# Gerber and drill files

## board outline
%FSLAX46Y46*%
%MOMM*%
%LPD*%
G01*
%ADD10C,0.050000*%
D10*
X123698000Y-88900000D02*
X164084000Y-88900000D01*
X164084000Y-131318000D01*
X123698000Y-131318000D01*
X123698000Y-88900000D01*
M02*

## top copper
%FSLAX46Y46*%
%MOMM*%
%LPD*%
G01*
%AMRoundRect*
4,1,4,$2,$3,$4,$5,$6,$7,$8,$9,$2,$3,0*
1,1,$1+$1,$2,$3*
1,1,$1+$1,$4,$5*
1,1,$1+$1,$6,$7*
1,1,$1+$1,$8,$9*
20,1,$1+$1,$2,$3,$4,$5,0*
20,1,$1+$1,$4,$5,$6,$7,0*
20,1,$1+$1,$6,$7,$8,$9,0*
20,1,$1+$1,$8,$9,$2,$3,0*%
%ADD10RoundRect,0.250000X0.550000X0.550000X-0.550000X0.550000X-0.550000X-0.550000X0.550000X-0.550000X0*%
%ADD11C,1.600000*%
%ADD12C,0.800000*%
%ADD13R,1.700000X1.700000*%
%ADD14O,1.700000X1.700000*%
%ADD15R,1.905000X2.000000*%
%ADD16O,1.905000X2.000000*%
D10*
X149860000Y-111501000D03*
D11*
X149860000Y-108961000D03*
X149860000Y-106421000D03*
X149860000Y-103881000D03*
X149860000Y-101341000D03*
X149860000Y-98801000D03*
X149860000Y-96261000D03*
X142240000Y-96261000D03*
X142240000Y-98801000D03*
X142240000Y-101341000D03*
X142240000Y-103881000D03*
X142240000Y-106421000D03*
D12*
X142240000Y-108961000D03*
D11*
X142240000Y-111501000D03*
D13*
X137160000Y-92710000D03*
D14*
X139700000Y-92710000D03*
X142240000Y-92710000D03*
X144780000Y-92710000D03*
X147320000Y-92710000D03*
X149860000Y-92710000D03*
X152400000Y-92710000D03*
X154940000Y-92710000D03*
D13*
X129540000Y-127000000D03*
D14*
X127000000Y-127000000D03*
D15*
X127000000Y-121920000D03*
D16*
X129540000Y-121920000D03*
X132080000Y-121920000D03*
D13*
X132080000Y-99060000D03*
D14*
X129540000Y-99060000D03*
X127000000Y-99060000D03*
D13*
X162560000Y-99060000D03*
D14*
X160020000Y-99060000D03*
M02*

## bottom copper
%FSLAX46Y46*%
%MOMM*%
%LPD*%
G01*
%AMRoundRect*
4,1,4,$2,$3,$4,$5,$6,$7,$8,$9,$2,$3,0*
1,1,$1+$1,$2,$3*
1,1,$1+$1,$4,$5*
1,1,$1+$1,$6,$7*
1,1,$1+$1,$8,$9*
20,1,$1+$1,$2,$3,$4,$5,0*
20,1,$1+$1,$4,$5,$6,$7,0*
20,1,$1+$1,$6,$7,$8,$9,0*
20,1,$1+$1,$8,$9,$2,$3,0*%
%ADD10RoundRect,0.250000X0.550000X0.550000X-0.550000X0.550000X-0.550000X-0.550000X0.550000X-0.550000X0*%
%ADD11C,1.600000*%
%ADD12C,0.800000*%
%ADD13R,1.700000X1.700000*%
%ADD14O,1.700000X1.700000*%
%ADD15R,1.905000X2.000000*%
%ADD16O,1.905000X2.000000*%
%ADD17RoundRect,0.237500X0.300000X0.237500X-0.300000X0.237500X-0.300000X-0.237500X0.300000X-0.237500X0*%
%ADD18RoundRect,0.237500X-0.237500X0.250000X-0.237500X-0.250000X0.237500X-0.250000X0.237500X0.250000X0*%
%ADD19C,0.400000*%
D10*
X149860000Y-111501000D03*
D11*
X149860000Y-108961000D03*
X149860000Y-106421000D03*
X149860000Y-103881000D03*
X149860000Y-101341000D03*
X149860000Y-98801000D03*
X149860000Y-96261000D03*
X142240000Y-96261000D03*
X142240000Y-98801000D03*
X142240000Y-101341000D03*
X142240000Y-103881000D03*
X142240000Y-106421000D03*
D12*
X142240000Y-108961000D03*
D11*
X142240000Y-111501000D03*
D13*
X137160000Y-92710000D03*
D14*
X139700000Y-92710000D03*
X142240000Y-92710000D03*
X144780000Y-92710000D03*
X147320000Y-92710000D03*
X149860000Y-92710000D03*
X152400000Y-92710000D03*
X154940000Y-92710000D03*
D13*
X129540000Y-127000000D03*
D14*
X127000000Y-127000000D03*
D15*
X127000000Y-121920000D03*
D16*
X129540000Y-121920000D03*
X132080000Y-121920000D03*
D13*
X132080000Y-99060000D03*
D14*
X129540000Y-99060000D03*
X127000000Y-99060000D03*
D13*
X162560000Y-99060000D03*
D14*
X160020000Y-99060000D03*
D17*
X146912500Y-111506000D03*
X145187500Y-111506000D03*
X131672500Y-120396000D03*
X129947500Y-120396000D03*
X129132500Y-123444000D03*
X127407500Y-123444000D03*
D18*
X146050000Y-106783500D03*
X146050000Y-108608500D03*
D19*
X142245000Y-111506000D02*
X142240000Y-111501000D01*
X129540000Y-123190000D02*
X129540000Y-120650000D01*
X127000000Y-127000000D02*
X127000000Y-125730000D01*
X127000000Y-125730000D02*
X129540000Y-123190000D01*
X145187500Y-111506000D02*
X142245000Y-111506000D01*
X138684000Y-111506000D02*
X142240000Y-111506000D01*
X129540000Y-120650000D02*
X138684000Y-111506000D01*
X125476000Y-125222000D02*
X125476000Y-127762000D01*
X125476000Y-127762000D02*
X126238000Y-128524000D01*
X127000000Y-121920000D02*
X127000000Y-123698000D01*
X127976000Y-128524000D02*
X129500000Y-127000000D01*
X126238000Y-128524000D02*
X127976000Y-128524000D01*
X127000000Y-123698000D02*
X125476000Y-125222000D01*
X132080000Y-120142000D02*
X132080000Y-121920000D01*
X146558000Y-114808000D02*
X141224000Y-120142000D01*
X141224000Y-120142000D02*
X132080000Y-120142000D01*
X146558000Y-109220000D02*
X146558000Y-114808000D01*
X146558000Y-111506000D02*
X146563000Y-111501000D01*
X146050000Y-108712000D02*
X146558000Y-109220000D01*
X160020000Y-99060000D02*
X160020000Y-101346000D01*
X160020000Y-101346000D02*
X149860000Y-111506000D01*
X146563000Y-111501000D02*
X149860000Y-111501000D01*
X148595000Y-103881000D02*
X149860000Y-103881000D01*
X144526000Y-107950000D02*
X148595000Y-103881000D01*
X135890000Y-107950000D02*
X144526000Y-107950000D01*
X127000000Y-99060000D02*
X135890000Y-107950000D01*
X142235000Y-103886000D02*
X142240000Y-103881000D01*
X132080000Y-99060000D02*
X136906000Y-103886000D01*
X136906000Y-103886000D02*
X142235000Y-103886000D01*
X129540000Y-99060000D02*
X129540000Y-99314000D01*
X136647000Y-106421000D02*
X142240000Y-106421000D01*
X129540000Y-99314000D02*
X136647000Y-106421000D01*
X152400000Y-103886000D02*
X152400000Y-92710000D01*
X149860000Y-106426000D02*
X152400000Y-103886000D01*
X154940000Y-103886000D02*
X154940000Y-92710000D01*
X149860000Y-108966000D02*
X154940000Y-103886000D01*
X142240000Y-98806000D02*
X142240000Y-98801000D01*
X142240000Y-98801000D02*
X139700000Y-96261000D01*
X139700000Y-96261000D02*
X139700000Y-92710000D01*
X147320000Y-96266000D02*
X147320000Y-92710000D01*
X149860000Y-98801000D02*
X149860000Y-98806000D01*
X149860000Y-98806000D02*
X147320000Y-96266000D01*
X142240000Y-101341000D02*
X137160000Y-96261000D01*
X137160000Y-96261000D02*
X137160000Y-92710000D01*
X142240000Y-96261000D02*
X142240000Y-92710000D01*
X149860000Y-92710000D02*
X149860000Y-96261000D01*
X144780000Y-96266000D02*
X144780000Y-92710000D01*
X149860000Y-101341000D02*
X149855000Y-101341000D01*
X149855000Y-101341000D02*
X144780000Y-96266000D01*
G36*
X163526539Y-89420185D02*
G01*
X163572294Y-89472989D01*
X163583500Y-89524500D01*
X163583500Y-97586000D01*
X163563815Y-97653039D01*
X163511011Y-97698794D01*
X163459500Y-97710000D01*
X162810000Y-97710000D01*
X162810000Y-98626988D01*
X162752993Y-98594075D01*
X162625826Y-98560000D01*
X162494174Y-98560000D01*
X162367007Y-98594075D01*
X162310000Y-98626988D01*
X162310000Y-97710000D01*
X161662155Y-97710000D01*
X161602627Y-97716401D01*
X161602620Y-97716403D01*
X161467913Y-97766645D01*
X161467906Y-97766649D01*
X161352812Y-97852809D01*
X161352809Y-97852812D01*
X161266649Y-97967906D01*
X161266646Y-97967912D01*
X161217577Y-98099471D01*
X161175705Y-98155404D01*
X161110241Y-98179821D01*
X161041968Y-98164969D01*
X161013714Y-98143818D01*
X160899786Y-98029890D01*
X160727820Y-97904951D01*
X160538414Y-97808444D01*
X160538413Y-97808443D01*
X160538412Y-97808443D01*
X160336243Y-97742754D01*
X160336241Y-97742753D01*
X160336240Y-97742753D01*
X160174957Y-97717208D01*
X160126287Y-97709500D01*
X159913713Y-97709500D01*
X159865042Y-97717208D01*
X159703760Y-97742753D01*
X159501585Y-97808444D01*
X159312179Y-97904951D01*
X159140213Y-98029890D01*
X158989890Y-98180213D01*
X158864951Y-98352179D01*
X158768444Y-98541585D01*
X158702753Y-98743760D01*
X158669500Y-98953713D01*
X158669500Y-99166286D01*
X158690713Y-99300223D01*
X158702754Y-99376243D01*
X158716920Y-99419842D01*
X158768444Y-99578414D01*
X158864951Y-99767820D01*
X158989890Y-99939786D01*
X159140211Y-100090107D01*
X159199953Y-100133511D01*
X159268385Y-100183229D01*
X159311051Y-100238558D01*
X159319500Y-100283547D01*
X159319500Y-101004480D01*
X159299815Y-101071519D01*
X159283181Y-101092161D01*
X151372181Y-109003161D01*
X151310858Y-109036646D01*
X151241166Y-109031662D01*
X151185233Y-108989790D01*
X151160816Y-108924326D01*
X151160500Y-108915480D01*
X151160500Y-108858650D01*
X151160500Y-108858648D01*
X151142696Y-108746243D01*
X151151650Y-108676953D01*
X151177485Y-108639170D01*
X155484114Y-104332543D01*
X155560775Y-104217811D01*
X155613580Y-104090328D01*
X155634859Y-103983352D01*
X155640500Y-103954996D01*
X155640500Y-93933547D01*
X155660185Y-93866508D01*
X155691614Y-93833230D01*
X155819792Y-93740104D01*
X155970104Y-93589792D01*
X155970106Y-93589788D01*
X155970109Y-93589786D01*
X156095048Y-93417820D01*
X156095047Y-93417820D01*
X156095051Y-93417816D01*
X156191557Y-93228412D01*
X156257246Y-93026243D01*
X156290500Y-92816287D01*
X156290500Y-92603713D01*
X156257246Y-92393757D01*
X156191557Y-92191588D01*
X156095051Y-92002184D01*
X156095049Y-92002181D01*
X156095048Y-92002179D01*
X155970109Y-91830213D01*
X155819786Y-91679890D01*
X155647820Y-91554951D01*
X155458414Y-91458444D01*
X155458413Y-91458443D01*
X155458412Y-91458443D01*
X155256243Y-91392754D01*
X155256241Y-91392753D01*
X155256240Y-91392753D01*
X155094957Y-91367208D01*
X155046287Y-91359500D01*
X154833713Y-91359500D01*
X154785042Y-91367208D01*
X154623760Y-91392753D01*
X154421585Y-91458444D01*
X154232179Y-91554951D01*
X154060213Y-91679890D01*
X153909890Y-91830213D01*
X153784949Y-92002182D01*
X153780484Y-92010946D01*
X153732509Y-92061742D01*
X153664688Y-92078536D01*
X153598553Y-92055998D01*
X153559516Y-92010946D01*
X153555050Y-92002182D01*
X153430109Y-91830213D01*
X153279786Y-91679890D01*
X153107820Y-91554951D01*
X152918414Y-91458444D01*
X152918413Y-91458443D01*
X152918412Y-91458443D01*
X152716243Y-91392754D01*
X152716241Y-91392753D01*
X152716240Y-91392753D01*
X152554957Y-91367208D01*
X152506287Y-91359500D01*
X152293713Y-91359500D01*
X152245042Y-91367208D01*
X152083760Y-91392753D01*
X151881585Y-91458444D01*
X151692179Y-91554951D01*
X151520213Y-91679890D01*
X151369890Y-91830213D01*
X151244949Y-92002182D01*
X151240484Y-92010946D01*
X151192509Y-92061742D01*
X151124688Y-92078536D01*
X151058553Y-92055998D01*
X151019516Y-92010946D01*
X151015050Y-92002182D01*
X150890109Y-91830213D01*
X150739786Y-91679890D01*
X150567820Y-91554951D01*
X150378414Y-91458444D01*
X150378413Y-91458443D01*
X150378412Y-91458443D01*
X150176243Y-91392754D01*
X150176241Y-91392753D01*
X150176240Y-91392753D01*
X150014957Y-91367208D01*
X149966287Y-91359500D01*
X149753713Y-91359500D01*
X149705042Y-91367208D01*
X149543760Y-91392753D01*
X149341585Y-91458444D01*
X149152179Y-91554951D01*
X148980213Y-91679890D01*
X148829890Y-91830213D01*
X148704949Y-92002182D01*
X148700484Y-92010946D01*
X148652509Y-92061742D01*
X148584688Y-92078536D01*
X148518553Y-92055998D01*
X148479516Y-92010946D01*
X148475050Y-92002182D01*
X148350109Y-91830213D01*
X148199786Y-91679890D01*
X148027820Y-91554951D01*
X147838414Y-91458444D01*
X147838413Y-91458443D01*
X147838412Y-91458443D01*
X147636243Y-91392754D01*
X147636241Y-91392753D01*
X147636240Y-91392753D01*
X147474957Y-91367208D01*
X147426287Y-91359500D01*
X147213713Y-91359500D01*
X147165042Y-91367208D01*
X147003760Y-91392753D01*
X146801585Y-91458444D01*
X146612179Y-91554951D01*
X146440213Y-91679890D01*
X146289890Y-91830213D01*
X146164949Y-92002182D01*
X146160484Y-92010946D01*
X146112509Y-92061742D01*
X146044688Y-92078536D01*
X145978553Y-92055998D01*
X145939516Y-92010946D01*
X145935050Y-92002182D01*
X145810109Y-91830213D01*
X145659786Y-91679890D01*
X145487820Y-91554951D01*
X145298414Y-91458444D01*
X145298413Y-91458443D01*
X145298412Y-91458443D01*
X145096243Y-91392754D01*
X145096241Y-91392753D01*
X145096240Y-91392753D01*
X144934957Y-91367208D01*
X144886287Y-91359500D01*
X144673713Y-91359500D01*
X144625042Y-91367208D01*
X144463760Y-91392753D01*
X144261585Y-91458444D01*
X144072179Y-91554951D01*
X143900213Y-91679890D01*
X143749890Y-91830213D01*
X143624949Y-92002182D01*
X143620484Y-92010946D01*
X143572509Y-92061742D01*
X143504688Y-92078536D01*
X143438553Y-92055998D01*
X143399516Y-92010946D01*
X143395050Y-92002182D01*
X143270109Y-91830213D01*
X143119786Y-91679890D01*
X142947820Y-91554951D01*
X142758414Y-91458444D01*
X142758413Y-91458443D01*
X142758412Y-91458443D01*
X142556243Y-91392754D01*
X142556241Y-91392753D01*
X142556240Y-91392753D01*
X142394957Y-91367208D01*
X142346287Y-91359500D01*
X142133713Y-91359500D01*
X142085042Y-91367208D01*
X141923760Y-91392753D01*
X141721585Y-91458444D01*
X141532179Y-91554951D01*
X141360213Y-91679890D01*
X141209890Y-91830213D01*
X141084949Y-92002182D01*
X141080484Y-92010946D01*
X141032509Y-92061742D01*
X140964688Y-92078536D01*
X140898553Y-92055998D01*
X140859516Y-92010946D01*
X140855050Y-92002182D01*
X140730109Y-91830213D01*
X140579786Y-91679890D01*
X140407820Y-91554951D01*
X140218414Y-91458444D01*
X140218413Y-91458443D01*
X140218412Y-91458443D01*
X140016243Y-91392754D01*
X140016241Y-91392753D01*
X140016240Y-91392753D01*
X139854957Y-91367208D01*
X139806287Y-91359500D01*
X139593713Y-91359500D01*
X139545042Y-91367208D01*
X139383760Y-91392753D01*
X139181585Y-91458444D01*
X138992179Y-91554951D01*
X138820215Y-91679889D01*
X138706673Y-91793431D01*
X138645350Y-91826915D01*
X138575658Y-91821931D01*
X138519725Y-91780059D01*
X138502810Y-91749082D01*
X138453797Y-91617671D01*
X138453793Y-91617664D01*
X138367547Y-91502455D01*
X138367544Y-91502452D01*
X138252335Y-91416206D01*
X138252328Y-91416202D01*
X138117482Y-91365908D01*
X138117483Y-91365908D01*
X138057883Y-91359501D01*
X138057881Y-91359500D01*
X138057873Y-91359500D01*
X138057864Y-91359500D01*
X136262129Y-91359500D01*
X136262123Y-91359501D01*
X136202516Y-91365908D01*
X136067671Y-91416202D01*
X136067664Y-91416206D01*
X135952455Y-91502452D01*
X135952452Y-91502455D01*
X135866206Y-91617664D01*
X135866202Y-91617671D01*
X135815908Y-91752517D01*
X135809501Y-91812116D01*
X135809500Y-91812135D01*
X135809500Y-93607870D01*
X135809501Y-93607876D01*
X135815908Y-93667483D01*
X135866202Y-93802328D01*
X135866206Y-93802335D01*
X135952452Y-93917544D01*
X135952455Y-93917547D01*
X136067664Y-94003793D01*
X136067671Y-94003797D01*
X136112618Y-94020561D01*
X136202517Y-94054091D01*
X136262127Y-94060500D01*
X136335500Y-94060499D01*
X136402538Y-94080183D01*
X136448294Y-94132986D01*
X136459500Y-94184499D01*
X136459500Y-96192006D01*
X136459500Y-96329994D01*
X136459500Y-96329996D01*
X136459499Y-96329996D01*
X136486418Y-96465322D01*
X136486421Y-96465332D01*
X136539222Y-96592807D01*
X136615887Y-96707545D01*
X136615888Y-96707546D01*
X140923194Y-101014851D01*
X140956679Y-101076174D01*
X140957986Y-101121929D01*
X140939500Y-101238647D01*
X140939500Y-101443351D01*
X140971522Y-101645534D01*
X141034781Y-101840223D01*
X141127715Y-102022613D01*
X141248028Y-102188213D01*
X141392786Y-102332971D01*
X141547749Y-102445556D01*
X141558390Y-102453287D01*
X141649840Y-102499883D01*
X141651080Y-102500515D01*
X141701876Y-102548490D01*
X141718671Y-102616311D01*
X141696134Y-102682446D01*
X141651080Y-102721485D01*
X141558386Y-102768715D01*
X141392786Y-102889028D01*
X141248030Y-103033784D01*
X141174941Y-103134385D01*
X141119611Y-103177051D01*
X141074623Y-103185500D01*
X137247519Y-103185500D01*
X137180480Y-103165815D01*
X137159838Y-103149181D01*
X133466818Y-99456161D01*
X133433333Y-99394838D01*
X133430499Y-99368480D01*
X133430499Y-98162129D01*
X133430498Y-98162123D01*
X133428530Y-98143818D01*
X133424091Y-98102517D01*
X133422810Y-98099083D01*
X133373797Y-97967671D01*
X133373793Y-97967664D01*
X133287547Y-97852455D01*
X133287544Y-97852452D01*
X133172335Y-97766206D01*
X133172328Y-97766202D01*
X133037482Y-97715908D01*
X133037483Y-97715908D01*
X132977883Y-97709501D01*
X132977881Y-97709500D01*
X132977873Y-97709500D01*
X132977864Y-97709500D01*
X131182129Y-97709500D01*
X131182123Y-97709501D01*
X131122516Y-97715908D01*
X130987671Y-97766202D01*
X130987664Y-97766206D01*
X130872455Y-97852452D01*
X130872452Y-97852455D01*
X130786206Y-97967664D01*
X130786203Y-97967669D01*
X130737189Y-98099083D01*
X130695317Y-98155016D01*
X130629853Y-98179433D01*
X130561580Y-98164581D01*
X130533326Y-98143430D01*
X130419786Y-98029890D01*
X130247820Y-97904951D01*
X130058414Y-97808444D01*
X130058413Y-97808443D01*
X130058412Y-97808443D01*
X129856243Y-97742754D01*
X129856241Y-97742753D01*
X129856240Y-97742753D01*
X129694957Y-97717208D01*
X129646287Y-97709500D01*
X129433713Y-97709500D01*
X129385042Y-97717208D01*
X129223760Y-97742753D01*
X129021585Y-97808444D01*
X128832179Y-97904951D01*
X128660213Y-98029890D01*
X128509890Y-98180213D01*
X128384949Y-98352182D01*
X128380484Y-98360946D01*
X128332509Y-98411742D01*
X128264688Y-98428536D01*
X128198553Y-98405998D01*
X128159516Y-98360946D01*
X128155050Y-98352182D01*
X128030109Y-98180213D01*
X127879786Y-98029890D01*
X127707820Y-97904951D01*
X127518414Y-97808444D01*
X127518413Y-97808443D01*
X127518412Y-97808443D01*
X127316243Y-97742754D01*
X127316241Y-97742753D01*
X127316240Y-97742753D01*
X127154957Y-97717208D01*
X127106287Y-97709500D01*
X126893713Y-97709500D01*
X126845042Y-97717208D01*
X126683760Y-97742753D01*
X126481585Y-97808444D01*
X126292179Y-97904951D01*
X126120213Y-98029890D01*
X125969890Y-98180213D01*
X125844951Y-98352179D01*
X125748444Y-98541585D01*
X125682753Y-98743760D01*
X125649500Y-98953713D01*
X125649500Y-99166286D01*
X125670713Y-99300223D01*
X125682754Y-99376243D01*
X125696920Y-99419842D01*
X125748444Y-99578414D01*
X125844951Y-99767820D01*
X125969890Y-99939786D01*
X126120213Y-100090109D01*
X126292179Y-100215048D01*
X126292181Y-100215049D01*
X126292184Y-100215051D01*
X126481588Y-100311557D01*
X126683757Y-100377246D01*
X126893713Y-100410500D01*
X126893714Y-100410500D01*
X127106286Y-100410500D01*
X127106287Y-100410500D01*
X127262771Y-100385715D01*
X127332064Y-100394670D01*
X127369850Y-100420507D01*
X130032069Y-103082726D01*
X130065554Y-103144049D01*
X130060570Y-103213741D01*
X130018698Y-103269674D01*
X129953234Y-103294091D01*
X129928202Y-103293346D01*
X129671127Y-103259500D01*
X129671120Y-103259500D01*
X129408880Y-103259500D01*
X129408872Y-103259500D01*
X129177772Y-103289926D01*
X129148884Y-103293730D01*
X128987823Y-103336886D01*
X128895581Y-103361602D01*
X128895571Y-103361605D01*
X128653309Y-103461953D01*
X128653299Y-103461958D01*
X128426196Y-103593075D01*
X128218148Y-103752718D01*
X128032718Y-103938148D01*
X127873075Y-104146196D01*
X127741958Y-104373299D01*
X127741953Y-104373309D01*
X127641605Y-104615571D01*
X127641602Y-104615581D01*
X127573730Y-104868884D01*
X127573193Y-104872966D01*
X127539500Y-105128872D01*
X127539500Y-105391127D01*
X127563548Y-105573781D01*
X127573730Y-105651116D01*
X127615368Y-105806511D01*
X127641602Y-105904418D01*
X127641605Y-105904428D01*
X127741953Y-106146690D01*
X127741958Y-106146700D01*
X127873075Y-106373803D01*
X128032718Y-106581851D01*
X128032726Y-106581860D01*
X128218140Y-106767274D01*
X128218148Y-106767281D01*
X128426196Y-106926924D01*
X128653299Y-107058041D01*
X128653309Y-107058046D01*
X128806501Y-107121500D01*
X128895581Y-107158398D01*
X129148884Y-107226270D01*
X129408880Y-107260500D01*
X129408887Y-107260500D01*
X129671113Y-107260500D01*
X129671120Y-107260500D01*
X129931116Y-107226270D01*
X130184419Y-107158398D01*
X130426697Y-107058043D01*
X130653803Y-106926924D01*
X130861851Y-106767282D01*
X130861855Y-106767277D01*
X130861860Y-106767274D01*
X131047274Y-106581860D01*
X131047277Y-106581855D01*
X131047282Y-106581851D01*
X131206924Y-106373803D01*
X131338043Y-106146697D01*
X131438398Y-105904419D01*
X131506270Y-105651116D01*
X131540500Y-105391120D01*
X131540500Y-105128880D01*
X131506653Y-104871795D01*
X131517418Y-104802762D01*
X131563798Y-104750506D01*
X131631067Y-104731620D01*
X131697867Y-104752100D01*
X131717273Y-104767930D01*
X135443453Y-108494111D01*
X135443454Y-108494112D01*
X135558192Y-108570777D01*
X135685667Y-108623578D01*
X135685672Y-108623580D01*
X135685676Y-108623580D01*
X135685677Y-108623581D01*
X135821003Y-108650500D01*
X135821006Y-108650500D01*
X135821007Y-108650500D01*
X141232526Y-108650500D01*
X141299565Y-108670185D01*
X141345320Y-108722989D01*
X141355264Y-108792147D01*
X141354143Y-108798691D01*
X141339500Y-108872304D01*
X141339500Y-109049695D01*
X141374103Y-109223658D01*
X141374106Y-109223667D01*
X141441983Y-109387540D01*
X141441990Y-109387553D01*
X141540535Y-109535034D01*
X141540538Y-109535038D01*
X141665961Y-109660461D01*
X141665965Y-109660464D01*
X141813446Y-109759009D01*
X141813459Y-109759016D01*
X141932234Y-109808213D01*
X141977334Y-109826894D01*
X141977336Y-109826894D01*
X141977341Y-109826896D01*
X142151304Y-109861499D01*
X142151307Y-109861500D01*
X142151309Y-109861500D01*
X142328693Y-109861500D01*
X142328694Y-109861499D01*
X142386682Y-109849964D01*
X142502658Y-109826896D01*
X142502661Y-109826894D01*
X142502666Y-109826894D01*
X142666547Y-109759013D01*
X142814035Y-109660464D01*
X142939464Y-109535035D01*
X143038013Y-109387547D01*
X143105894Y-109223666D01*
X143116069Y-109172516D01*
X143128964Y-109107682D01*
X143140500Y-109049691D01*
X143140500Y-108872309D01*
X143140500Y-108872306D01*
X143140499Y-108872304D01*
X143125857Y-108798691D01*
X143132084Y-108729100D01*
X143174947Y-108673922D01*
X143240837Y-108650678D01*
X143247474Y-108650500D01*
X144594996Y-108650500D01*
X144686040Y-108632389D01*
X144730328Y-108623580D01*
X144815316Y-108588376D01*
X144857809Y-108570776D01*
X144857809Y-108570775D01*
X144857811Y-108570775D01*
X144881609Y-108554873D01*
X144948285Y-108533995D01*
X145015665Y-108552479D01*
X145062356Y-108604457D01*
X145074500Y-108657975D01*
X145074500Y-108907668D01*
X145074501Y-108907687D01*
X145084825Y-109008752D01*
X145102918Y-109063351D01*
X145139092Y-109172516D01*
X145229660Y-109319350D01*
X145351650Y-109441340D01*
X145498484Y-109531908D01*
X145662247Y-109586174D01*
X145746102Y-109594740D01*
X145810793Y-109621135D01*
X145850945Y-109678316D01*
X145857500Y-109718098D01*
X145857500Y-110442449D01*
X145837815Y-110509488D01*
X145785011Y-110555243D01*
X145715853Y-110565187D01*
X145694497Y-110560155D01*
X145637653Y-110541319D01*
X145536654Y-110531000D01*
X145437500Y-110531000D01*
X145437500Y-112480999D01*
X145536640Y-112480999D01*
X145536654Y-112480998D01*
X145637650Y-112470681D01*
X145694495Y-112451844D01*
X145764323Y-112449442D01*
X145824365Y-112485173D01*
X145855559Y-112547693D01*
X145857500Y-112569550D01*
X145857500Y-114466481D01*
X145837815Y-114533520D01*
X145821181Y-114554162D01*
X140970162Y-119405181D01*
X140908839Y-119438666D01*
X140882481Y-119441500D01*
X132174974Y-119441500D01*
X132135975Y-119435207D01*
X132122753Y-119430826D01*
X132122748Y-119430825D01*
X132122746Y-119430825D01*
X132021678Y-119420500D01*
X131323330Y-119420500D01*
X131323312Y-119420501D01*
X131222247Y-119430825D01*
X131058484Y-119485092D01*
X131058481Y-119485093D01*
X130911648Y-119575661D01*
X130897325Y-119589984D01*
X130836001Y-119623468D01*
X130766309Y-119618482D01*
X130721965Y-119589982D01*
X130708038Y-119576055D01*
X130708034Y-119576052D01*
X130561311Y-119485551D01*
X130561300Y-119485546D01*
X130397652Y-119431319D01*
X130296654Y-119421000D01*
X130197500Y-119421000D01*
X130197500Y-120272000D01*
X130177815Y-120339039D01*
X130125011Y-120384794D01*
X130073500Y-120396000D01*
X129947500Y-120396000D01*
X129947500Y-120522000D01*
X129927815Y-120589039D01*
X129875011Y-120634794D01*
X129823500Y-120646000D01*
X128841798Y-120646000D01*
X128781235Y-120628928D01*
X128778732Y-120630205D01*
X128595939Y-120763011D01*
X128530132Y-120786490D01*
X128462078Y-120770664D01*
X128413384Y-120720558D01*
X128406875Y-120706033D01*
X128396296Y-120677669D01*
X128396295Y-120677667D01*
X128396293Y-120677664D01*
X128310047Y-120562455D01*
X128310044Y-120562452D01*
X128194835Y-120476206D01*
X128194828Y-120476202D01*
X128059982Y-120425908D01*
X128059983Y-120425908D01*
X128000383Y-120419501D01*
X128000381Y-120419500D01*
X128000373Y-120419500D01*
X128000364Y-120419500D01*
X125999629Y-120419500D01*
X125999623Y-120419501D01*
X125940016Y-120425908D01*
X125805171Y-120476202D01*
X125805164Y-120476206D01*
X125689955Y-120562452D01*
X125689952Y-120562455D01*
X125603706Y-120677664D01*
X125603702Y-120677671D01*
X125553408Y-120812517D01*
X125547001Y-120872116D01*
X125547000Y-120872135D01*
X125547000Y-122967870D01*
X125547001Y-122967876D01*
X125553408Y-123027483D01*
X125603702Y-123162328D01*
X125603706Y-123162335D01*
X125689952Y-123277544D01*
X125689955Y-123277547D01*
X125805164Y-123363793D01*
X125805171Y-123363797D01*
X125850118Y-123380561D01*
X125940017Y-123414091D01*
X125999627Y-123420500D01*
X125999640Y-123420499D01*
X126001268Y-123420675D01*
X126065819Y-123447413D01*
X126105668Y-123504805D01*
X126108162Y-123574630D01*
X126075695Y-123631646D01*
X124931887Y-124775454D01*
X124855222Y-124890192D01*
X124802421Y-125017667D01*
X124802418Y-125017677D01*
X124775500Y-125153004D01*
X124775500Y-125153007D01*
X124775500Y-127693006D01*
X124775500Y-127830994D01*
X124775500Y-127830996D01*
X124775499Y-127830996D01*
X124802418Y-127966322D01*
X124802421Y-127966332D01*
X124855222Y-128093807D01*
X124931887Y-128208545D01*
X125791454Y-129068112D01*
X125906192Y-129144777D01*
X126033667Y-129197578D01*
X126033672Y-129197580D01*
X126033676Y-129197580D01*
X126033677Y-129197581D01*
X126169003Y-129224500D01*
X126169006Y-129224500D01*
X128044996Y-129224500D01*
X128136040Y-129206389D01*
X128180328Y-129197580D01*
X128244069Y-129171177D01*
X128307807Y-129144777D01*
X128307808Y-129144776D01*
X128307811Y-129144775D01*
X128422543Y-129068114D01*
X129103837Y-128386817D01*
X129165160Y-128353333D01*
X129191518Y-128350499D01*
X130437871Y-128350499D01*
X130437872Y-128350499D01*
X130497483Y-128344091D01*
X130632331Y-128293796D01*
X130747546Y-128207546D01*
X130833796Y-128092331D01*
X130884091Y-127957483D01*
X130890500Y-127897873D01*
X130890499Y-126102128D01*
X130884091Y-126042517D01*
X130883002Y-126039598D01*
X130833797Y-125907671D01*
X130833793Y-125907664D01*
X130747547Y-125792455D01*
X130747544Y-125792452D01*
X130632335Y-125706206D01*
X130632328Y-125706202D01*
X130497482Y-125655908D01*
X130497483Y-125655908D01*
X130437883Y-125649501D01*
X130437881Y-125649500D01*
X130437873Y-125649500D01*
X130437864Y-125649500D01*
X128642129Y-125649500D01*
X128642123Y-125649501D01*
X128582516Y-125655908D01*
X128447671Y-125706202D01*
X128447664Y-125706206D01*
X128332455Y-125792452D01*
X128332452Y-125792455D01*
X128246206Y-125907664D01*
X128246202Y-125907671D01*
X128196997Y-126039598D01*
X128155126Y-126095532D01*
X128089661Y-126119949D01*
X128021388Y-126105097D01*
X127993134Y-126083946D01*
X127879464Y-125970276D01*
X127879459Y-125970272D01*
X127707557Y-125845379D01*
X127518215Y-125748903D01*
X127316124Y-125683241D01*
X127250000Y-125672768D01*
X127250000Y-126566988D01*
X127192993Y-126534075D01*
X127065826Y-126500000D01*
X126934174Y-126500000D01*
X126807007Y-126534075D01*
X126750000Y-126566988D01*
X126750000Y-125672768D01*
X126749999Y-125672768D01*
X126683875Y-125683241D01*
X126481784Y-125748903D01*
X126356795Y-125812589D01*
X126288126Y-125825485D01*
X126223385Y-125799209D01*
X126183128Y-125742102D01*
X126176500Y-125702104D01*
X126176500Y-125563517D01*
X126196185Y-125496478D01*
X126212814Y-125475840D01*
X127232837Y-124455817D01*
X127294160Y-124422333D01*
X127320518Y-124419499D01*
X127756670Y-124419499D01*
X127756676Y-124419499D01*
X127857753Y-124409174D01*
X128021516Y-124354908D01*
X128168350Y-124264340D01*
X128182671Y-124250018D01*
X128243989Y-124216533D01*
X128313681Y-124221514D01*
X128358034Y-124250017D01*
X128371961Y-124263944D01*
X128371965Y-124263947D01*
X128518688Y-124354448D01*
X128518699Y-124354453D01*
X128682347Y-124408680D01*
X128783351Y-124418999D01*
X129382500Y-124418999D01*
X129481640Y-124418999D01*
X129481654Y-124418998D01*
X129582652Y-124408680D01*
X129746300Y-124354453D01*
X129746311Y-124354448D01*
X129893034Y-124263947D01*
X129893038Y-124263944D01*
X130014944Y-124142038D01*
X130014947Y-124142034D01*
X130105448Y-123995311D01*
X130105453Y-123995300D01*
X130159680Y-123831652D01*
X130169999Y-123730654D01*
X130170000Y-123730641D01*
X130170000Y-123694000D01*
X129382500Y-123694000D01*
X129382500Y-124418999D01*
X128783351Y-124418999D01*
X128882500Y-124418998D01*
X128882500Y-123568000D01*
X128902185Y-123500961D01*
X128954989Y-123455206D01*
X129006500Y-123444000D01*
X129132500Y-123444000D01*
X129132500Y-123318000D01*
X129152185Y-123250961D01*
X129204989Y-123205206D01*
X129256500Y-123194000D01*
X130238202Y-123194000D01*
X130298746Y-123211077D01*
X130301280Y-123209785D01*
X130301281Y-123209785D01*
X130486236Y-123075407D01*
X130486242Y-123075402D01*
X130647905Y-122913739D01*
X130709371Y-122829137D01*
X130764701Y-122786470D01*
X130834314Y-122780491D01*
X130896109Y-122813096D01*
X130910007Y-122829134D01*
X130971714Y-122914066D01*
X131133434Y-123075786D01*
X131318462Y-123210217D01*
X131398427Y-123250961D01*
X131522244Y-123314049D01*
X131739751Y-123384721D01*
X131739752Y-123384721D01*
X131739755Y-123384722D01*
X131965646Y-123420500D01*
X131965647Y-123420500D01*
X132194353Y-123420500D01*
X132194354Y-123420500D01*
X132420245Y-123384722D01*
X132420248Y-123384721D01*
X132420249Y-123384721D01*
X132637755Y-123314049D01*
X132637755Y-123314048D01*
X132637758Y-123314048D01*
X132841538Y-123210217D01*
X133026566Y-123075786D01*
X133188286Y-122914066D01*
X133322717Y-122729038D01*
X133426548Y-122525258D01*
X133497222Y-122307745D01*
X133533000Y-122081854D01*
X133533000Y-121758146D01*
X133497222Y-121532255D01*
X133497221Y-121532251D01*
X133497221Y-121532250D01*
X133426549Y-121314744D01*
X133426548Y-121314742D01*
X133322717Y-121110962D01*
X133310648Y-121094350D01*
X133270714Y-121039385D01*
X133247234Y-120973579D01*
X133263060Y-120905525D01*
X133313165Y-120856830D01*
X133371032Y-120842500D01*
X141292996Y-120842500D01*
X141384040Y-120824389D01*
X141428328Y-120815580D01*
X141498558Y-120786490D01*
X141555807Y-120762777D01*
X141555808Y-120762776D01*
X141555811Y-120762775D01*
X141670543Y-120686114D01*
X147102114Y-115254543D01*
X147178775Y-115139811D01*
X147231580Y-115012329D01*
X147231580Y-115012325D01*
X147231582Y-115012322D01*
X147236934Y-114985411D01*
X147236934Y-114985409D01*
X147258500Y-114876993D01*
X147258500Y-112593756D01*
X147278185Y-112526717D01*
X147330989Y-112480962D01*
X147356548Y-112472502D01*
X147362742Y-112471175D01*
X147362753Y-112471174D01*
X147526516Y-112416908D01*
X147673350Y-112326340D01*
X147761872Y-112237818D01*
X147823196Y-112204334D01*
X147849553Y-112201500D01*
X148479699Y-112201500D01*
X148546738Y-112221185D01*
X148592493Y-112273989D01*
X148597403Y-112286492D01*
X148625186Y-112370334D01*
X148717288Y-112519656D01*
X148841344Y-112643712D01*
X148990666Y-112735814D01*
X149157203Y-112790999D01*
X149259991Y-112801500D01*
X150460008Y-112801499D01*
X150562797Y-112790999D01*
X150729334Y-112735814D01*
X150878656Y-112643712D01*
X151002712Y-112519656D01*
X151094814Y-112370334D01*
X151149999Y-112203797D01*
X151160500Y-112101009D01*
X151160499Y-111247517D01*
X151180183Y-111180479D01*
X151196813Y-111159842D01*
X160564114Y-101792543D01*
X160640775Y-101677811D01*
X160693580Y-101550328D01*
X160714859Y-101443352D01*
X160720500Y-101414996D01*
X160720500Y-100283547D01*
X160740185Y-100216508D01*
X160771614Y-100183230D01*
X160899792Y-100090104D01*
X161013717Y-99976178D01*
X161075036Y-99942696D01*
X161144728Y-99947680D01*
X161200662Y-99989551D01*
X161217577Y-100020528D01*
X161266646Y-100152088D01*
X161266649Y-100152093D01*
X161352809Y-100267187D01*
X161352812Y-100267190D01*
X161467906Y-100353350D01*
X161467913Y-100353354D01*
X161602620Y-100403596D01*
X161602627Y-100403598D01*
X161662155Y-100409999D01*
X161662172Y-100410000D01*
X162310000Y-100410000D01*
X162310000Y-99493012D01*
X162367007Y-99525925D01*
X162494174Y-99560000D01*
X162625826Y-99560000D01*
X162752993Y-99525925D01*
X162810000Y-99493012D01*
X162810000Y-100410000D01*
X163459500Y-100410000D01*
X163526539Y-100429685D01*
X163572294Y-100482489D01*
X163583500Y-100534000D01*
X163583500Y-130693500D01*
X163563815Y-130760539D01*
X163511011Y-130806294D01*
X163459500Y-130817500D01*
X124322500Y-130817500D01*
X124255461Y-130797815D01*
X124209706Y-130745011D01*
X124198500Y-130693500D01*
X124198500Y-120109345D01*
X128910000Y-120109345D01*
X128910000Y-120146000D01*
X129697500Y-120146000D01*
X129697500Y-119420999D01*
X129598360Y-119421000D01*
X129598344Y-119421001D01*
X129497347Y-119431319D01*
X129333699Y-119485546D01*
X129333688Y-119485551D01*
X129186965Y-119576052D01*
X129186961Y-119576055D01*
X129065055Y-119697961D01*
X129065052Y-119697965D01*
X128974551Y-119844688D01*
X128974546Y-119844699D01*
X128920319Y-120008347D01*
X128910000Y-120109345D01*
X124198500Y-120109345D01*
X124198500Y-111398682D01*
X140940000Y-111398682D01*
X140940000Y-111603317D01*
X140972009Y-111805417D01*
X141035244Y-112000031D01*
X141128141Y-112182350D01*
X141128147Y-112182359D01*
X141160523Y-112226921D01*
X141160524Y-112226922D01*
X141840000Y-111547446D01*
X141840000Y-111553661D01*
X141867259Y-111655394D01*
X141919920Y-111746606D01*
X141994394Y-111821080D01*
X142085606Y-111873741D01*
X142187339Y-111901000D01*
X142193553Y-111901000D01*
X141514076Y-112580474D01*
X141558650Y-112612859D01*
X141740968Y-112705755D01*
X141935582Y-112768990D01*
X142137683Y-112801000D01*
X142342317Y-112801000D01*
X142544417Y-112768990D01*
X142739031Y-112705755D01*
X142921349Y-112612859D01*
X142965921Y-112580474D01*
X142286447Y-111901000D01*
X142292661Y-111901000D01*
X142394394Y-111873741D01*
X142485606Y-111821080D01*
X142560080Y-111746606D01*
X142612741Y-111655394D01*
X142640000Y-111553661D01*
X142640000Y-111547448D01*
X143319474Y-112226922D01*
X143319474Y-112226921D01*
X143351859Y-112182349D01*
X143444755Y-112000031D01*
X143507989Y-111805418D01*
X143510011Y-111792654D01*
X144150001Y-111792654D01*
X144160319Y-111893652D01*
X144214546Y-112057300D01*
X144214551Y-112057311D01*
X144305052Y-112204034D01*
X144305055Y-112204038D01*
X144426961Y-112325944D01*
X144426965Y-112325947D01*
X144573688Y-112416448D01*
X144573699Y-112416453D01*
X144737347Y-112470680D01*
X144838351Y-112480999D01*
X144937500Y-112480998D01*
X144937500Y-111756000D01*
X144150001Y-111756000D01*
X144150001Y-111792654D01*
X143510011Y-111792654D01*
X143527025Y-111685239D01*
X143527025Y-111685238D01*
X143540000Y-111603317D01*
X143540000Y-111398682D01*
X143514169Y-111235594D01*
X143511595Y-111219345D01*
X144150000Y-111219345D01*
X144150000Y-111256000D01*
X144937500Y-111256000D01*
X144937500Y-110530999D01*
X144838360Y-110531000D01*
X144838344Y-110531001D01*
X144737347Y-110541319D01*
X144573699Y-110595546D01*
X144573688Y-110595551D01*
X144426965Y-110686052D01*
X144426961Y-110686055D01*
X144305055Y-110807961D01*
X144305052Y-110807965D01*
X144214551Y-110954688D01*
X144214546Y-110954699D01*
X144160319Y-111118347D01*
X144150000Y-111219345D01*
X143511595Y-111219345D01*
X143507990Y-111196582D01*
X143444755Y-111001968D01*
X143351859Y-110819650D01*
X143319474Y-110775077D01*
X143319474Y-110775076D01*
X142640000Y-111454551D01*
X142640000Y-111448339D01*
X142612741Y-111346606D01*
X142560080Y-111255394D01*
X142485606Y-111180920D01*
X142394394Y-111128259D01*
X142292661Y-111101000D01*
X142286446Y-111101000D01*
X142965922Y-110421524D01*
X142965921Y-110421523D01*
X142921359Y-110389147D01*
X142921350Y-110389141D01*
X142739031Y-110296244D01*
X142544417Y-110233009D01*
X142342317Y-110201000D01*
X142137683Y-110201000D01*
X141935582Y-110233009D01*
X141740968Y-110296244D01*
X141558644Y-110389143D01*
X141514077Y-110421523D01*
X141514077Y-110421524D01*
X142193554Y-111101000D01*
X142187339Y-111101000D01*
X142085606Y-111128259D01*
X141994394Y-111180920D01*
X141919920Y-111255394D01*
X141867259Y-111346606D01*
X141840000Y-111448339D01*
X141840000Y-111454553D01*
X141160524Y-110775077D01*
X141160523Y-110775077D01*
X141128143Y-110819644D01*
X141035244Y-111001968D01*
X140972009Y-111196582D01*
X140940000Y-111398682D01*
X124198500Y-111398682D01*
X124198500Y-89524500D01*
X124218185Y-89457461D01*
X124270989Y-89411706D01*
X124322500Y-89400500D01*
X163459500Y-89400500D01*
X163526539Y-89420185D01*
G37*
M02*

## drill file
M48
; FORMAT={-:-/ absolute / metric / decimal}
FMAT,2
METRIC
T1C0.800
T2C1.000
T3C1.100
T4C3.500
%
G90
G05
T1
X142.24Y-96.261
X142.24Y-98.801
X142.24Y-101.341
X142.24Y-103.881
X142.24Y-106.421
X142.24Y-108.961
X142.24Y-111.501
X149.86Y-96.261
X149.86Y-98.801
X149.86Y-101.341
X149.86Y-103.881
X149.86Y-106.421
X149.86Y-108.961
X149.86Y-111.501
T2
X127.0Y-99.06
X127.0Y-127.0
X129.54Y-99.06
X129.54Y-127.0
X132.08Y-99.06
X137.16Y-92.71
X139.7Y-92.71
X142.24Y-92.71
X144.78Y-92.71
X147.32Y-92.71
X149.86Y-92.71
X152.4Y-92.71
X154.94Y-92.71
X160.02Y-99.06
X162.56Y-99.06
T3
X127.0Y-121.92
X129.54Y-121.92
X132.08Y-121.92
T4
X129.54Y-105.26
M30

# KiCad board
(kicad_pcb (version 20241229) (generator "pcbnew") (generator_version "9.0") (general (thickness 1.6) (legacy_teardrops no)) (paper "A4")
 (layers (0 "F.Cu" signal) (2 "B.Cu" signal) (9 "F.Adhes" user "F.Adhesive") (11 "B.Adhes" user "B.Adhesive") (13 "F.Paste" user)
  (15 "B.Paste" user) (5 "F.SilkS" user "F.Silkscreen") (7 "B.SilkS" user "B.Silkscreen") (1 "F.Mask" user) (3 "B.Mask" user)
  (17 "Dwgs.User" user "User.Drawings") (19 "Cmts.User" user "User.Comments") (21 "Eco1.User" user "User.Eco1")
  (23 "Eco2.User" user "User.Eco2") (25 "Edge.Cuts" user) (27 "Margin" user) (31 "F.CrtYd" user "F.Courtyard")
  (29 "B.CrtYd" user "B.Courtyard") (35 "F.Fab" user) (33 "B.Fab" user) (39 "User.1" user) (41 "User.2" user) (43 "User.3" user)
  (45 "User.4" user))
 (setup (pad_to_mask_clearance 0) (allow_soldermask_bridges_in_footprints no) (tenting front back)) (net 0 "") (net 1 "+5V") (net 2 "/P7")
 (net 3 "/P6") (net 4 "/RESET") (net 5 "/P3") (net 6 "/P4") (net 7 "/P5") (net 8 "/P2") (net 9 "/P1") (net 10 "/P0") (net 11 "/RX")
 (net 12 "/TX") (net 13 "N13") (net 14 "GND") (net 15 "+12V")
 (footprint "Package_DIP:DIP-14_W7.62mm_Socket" (layer "F.Cu") (at 149.86 111.501 180)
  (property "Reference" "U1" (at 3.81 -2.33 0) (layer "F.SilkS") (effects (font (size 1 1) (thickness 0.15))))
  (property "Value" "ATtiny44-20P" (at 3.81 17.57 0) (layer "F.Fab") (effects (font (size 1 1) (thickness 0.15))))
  (pad "1" thru_hole roundrect (at 0 0 180) (size 1.6 1.6) (drill 0.8) (layers "*.Cu" "*.Mask") (remove_unused_layers no)
   (roundrect_rratio 0.15625) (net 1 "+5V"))
  (pad "2" thru_hole circle (at 0 2.54 180) (size 1.6 1.6) (drill 0.8) (layers "*.Cu" "*.Mask") (remove_unused_layers no) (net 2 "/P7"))
  (pad "3" thru_hole circle (at 0 5.08 180) (size 1.6 1.6) (drill 0.8) (layers "*.Cu" "*.Mask") (remove_unused_layers no) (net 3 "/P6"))
  (pad "4" thru_hole circle (at 0 7.62 180) (size 1.6 1.6) (drill 0.8) (layers "*.Cu" "*.Mask") (remove_unused_layers no) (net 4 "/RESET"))
  (pad "5" thru_hole circle (at 0 10.16 180) (size 1.6 1.6) (drill 0.8) (layers "*.Cu" "*.Mask") (remove_unused_layers no) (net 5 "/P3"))
  (pad "6" thru_hole circle (at 0 12.7 180) (size 1.6 1.6) (drill 0.8) (layers "*.Cu" "*.Mask") (remove_unused_layers no) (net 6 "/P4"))
  (pad "7" thru_hole circle (at 0 15.24 180) (size 1.6 1.6) (drill 0.8) (layers "*.Cu" "*.Mask") (remove_unused_layers no) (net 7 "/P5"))
  (pad "8" thru_hole circle (at 7.62 15.24 180) (size 1.6 1.6) (drill 0.8) (layers "*.Cu" "*.Mask") (remove_unused_layers no) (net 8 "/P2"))
  (pad "9" thru_hole circle (at 7.62 12.7 180) (size 1.6 1.6) (drill 0.8) (layers "*.Cu" "*.Mask") (remove_unused_layers no) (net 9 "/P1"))
  (pad "10" thru_hole circle (at 7.62 10.16 180) (size 1.6 1.6) (drill 0.8) (layers "*.Cu" "*.Mask") (remove_unused_layers no)
   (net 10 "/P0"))
  (pad "11" thru_hole circle (at 7.62 7.62 180) (size 1.6 1.6) (drill 0.8) (layers "*.Cu" "*.Mask") (remove_unused_layers no) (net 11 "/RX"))
  (pad "12" thru_hole circle (at 7.62 5.08 180) (size 1.6 1.6) (drill 0.8) (layers "*.Cu" "*.Mask") (remove_unused_layers no) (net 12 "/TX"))
  (pad "13" thru_hole circle (at 7.62 2.54 180) (size 0.8 0.8) (drill 0.8) (layers "*.Cu" "*.Mask") (remove_unused_layers no) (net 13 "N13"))
  (pad "14" thru_hole circle (at 7.62 0 180) (size 1.6 1.6) (drill 0.8) (layers "*.Cu" "*.Mask") (remove_unused_layers no) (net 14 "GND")))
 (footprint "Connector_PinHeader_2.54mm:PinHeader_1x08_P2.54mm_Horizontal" (layer "F.Cu") (at 137.16 92.71 90)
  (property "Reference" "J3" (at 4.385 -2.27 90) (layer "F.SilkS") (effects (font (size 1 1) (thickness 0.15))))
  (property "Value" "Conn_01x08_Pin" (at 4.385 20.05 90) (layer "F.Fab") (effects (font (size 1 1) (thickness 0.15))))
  (pad "1" thru_hole rect (at 0 0 90) (size 1.7 1.7) (drill 1) (layers "*.Cu" "*.Mask") (remove_unused_layers no) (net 10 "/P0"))
  (pad "2" thru_hole oval (at 0 2.54 90) (size 1.7 1.7) (drill 1) (layers "*.Cu" "*.Mask") (remove_unused_layers no) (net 9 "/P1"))
  (pad "3" thru_hole oval (at 0 5.08 90) (size 1.7 1.7) (drill 1) (layers "*.Cu" "*.Mask") (remove_unused_layers no) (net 8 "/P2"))
  (pad "4" thru_hole oval (at 0 7.62 90) (size 1.7 1.7) (drill 1) (layers "*.Cu" "*.Mask") (remove_unused_layers no) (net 5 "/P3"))
  (pad "5" thru_hole oval (at 0 10.16 90) (size 1.7 1.7) (drill 1) (layers "*.Cu" "*.Mask") (remove_unused_layers no) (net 6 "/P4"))
  (pad "6" thru_hole oval (at 0 12.7 90) (size 1.7 1.7) (drill 1) (layers "*.Cu" "*.Mask") (remove_unused_layers no) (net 7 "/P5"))
  (pad "7" thru_hole oval (at 0 15.24 90) (size 1.7 1.7) (drill 1) (layers "*.Cu" "*.Mask") (remove_unused_layers no) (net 3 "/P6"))
  (pad "8" thru_hole oval (at 0 17.78 90) (size 1.7 1.7) (drill 1) (layers "*.Cu" "*.Mask") (remove_unused_layers no) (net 2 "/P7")))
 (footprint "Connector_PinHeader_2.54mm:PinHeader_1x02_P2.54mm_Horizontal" (layer "F.Cu") (at 129.54 127 -90)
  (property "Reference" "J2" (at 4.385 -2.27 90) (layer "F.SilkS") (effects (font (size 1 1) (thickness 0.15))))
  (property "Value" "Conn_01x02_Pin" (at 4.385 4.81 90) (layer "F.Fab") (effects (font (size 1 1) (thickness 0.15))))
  (pad "1" thru_hole rect (at 0 0 270) (size 1.7 1.7) (drill 1) (layers "*.Cu" "*.Mask") (remove_unused_layers no) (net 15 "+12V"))
  (pad "2" thru_hole oval (at 0 2.54 270) (size 1.7 1.7) (drill 1) (layers "*.Cu" "*.Mask") (remove_unused_layers no) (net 14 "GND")))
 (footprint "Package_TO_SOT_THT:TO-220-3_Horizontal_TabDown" (layer "F.Cu") (at 127 121.92)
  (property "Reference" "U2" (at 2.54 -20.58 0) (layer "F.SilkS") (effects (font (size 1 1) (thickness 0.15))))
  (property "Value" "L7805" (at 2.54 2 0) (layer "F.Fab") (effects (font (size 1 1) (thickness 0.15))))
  (pad "" np_thru_hole circle (at 2.54 -16.66) (size 3.5 3.5) (drill 3.5) (layers "*.Cu" "*.Mask"))
  (pad "1" thru_hole rect (at 0 0) (size 1.905 2) (drill 1.1) (layers "*.Cu" "*.Mask") (remove_unused_layers no) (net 15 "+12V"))
  (pad "2" thru_hole oval (at 2.54 0) (size 1.905 2) (drill 1.1) (layers "*.Cu" "*.Mask") (remove_unused_layers no) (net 14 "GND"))
  (pad "3" thru_hole oval (at 5.08 0) (size 1.905 2) (drill 1.1) (layers "*.Cu" "*.Mask") (remove_unused_layers no) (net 1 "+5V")))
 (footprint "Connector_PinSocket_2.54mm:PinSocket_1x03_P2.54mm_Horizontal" (layer "F.Cu") (at 132.08 99.06 -90)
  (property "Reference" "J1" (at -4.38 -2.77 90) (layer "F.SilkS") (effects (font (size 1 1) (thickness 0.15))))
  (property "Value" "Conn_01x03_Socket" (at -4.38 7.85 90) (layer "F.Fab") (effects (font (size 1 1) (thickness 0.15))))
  (pad "1" thru_hole rect (at 0 0 270) (size 1.7 1.7) (drill 1) (layers "*.Cu" "*.Mask") (remove_unused_layers no) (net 11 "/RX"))
  (pad "2" thru_hole oval (at 0 2.54 270) (size 1.7 1.7) (drill 1) (layers "*.Cu" "*.Mask") (remove_unused_layers no) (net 12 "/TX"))
  (pad "3" thru_hole oval (at 0 5.08 270) (size 1.7 1.7) (drill 1) (layers "*.Cu" "*.Mask") (remove_unused_layers no) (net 4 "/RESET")))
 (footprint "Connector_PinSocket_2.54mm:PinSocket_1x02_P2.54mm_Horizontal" (layer "F.Cu") (at 162.56 99.06 -90)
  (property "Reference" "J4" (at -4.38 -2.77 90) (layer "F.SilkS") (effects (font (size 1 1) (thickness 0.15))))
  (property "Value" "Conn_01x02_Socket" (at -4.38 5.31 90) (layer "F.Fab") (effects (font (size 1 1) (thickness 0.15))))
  (pad "1" thru_hole rect (at 0 0 270) (size 1.7 1.7) (drill 1) (layers "*.Cu" "*.Mask") (remove_unused_layers no) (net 14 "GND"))
  (pad "2" thru_hole oval (at 0 2.54 270) (size 1.7 1.7) (drill 1) (layers "*.Cu" "*.Mask") (remove_unused_layers no) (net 1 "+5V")))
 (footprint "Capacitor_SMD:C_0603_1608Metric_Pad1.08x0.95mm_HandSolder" (layer "B.Cu") (at 146.05 111.506 180)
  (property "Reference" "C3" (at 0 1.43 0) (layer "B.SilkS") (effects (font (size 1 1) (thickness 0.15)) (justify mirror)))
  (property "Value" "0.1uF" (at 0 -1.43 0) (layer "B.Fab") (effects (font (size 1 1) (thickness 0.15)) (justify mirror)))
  (pad "1" smd roundrect (at -0.8625 0 180) (size 1.075 0.95) (layers "B.Cu" "B.Mask" "B.Paste") (roundrect_rratio 0.25) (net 1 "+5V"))
  (pad "2" smd roundrect (at 0.8625 0 180) (size 1.075 0.95) (layers "B.Cu" "B.Mask" "B.Paste") (roundrect_rratio 0.25) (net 14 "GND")))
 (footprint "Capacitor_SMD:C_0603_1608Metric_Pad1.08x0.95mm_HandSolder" (layer "B.Cu") (at 130.81 120.396 180)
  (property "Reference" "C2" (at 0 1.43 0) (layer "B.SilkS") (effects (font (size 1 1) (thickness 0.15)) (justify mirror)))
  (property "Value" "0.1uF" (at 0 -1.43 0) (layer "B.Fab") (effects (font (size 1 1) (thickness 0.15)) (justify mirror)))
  (pad "1" smd roundrect (at -0.8625 0 180) (size 1.075 0.95) (layers "B.Cu" "B.Mask" "B.Paste") (roundrect_rratio 0.25) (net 1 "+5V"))
  (pad "2" smd roundrect (at 0.8625 0 180) (size 1.075 0.95) (layers "B.Cu" "B.Mask" "B.Paste") (roundrect_rratio 0.25) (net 14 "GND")))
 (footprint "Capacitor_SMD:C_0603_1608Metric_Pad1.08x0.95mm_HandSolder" (layer "B.Cu") (at 128.27 123.444 180)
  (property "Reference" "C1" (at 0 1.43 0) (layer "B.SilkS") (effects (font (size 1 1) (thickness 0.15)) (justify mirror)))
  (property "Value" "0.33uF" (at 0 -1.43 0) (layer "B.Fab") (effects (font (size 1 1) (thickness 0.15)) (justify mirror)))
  (pad "1" smd roundrect (at -0.8625 0 180) (size 1.075 0.95) (layers "B.Cu" "B.Mask" "B.Paste") (roundrect_rratio 0.25) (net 14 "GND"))
  (pad "2" smd roundrect (at 0.8625 0 180) (size 1.075 0.95) (layers "B.Cu" "B.Mask" "B.Paste") (roundrect_rratio 0.25) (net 15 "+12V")))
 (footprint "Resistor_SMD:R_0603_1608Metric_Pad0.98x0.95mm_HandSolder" (layer "B.Cu") (at 146.05 107.696 -90)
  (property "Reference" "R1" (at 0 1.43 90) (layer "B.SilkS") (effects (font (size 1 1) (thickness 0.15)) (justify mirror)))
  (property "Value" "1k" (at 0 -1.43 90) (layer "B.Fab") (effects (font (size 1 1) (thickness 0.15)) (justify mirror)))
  (pad "1" smd roundrect (at -0.9125 0 270) (size 0.975 0.95) (layers "B.Cu" "B.Mask" "B.Paste") (roundrect_rratio 0.25) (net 4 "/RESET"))
  (pad "2" smd roundrect (at 0.9125 0 270) (size 0.975 0.95) (layers "B.Cu" "B.Mask" "B.Paste") (roundrect_rratio 0.25) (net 1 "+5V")))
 (gr_rect (start 123.698 88.9) (end 164.084 131.318) (stroke (width 0.05) (type default)) (fill no) (layer "Edge.Cuts"))
 (segment (start 142.245 111.506) (end 142.24 111.501) (width 0.4) (layer "B.Cu") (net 14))
 (segment (start 129.54 123.19) (end 129.54 120.65) (width 0.4) (layer "B.Cu") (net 14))
 (segment (start 127 127) (end 127 125.73) (width 0.4) (layer "B.Cu") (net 14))
 (segment (start 127 125.73) (end 129.54 123.19) (width 0.4) (layer "B.Cu") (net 14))
 (segment (start 145.1875 111.506) (end 142.245 111.506) (width 0.4) (layer "B.Cu") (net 14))
 (segment (start 138.684 111.506) (end 142.24 111.506) (width 0.4) (layer "B.Cu") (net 14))
 (segment (start 129.54 120.65) (end 138.684 111.506) (width 0.4) (layer "B.Cu") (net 14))
 (segment (start 125.476 125.222) (end 125.476 127.762) (width 0.4) (layer "B.Cu") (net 15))
 (segment (start 125.476 127.762) (end 126.238 128.524) (width 0.4) (layer "B.Cu") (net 15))
 (segment (start 127 121.92) (end 127 123.698) (width 0.4) (layer "B.Cu") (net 15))
 (segment (start 127.976 128.524) (end 129.5 127) (width 0.4) (layer "B.Cu") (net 15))
 (segment (start 126.238 128.524) (end 127.976 128.524) (width 0.4) (layer "B.Cu") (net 15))
 (segment (start 127 123.698) (end 125.476 125.222) (width 0.4) (layer "B.Cu") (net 15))
 (segment (start 132.08 120.142) (end 132.08 121.92) (width 0.4) (layer "B.Cu") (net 1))
 (segment (start 146.558 114.808) (end 141.224 120.142) (width 0.4) (layer "B.Cu") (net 1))
 (segment (start 141.224 120.142) (end 132.08 120.142) (width 0.4) (layer "B.Cu") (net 1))
 (segment (start 146.558 109.22) (end 146.558 114.808) (width 0.4) (layer "B.Cu") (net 1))
 (segment (start 146.558 111.506) (end 146.563 111.501) (width 0.4) (layer "B.Cu") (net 1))
 (segment (start 146.05 108.712) (end 146.558 109.22) (width 0.4) (layer "B.Cu") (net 1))
 (segment (start 160.02 99.06) (end 160.02 101.346) (width 0.4) (layer "B.Cu") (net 1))
 (segment (start 160.02 101.346) (end 149.86 111.506) (width 0.4) (layer "B.Cu") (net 1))
 (segment (start 146.563 111.501) (end 149.86 111.501) (width 0.4) (layer "B.Cu") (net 1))
 (segment (start 148.595 103.881) (end 149.86 103.881) (width 0.4) (layer "B.Cu") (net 4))
 (segment (start 144.526 107.95) (end 148.595 103.881) (width 0.4) (layer "B.Cu") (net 4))
 (segment (start 135.89 107.95) (end 144.526 107.95) (width 0.4) (layer "B.Cu") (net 4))
 (segment (start 127 99.06) (end 135.89 107.95) (width 0.4) (layer "B.Cu") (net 4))
 (segment (start 142.235 103.886) (end 142.24 103.881) (width 0.4) (layer "B.Cu") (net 11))
 (segment (start 132.08 99.06) (end 136.906 103.886) (width 0.4) (layer "B.Cu") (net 11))
 (segment (start 136.906 103.886) (end 142.235 103.886) (width 0.4) (layer "B.Cu") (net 11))
 (segment (start 129.54 99.06) (end 129.54 99.314) (width 0.4) (layer "B.Cu") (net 12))
 (segment (start 136.647 106.421) (end 142.24 106.421) (width 0.4) (layer "B.Cu") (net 12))
 (segment (start 129.54 99.314) (end 136.647 106.421) (width 0.4) (layer "B.Cu") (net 12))
 (segment (start 152.4 103.886) (end 152.4 92.71) (width 0.4) (layer "B.Cu") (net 3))
 (segment (start 149.86 106.426) (end 152.4 103.886) (width 0.4) (layer "B.Cu") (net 3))
 (segment (start 154.94 103.886) (end 154.94 92.71) (width 0.4) (layer "B.Cu") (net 2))
 (segment (start 149.86 108.966) (end 154.94 103.886) (width 0.4) (layer "B.Cu") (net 2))
 (segment (start 142.24 98.806) (end 142.24 98.801) (width 0.4) (layer "B.Cu") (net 9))
 (segment (start 142.24 98.801) (end 139.7 96.261) (width 0.4) (layer "B.Cu") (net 9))
 (segment (start 139.7 96.261) (end 139.7 92.71) (width 0.4) (layer "B.Cu") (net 9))
 (segment (start 147.32 96.266) (end 147.32 92.71) (width 0.4) (layer "B.Cu") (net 6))
 (segment (start 149.86 98.801) (end 149.86 98.806) (width 0.4) (layer "B.Cu") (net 6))
 (segment (start 149.86 98.806) (end 147.32 96.266) (width 0.4) (layer "B.Cu") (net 6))
 (segment (start 142.24 101.341) (end 137.16 96.261) (width 0.4) (layer "B.Cu") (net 10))
 (segment (start 137.16 96.261) (end 137.16 92.71) (width 0.4) (layer "B.Cu") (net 10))
 (segment (start 142.24 96.261) (end 142.24 92.71) (width 0.4) (layer "B.Cu") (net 8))
 (segment (start 149.86 92.71) (end 149.86 96.261) (width 0.4) (layer "B.Cu") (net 7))
 (segment (start 144.78 96.266) (end 144.78 92.71) (width 0.4) (layer "B.Cu") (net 5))
 (segment (start 149.86 101.341) (end 149.855 101.341) (width 0.4) (layer "B.Cu") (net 5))
 (segment (start 149.855 101.341) (end 144.78 96.266) (width 0.4) (layer "B.Cu") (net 5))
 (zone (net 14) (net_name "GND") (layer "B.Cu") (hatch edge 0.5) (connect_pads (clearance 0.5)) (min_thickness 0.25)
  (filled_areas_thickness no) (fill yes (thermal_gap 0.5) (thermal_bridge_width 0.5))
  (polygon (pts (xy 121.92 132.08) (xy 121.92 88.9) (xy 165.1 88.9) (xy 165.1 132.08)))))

